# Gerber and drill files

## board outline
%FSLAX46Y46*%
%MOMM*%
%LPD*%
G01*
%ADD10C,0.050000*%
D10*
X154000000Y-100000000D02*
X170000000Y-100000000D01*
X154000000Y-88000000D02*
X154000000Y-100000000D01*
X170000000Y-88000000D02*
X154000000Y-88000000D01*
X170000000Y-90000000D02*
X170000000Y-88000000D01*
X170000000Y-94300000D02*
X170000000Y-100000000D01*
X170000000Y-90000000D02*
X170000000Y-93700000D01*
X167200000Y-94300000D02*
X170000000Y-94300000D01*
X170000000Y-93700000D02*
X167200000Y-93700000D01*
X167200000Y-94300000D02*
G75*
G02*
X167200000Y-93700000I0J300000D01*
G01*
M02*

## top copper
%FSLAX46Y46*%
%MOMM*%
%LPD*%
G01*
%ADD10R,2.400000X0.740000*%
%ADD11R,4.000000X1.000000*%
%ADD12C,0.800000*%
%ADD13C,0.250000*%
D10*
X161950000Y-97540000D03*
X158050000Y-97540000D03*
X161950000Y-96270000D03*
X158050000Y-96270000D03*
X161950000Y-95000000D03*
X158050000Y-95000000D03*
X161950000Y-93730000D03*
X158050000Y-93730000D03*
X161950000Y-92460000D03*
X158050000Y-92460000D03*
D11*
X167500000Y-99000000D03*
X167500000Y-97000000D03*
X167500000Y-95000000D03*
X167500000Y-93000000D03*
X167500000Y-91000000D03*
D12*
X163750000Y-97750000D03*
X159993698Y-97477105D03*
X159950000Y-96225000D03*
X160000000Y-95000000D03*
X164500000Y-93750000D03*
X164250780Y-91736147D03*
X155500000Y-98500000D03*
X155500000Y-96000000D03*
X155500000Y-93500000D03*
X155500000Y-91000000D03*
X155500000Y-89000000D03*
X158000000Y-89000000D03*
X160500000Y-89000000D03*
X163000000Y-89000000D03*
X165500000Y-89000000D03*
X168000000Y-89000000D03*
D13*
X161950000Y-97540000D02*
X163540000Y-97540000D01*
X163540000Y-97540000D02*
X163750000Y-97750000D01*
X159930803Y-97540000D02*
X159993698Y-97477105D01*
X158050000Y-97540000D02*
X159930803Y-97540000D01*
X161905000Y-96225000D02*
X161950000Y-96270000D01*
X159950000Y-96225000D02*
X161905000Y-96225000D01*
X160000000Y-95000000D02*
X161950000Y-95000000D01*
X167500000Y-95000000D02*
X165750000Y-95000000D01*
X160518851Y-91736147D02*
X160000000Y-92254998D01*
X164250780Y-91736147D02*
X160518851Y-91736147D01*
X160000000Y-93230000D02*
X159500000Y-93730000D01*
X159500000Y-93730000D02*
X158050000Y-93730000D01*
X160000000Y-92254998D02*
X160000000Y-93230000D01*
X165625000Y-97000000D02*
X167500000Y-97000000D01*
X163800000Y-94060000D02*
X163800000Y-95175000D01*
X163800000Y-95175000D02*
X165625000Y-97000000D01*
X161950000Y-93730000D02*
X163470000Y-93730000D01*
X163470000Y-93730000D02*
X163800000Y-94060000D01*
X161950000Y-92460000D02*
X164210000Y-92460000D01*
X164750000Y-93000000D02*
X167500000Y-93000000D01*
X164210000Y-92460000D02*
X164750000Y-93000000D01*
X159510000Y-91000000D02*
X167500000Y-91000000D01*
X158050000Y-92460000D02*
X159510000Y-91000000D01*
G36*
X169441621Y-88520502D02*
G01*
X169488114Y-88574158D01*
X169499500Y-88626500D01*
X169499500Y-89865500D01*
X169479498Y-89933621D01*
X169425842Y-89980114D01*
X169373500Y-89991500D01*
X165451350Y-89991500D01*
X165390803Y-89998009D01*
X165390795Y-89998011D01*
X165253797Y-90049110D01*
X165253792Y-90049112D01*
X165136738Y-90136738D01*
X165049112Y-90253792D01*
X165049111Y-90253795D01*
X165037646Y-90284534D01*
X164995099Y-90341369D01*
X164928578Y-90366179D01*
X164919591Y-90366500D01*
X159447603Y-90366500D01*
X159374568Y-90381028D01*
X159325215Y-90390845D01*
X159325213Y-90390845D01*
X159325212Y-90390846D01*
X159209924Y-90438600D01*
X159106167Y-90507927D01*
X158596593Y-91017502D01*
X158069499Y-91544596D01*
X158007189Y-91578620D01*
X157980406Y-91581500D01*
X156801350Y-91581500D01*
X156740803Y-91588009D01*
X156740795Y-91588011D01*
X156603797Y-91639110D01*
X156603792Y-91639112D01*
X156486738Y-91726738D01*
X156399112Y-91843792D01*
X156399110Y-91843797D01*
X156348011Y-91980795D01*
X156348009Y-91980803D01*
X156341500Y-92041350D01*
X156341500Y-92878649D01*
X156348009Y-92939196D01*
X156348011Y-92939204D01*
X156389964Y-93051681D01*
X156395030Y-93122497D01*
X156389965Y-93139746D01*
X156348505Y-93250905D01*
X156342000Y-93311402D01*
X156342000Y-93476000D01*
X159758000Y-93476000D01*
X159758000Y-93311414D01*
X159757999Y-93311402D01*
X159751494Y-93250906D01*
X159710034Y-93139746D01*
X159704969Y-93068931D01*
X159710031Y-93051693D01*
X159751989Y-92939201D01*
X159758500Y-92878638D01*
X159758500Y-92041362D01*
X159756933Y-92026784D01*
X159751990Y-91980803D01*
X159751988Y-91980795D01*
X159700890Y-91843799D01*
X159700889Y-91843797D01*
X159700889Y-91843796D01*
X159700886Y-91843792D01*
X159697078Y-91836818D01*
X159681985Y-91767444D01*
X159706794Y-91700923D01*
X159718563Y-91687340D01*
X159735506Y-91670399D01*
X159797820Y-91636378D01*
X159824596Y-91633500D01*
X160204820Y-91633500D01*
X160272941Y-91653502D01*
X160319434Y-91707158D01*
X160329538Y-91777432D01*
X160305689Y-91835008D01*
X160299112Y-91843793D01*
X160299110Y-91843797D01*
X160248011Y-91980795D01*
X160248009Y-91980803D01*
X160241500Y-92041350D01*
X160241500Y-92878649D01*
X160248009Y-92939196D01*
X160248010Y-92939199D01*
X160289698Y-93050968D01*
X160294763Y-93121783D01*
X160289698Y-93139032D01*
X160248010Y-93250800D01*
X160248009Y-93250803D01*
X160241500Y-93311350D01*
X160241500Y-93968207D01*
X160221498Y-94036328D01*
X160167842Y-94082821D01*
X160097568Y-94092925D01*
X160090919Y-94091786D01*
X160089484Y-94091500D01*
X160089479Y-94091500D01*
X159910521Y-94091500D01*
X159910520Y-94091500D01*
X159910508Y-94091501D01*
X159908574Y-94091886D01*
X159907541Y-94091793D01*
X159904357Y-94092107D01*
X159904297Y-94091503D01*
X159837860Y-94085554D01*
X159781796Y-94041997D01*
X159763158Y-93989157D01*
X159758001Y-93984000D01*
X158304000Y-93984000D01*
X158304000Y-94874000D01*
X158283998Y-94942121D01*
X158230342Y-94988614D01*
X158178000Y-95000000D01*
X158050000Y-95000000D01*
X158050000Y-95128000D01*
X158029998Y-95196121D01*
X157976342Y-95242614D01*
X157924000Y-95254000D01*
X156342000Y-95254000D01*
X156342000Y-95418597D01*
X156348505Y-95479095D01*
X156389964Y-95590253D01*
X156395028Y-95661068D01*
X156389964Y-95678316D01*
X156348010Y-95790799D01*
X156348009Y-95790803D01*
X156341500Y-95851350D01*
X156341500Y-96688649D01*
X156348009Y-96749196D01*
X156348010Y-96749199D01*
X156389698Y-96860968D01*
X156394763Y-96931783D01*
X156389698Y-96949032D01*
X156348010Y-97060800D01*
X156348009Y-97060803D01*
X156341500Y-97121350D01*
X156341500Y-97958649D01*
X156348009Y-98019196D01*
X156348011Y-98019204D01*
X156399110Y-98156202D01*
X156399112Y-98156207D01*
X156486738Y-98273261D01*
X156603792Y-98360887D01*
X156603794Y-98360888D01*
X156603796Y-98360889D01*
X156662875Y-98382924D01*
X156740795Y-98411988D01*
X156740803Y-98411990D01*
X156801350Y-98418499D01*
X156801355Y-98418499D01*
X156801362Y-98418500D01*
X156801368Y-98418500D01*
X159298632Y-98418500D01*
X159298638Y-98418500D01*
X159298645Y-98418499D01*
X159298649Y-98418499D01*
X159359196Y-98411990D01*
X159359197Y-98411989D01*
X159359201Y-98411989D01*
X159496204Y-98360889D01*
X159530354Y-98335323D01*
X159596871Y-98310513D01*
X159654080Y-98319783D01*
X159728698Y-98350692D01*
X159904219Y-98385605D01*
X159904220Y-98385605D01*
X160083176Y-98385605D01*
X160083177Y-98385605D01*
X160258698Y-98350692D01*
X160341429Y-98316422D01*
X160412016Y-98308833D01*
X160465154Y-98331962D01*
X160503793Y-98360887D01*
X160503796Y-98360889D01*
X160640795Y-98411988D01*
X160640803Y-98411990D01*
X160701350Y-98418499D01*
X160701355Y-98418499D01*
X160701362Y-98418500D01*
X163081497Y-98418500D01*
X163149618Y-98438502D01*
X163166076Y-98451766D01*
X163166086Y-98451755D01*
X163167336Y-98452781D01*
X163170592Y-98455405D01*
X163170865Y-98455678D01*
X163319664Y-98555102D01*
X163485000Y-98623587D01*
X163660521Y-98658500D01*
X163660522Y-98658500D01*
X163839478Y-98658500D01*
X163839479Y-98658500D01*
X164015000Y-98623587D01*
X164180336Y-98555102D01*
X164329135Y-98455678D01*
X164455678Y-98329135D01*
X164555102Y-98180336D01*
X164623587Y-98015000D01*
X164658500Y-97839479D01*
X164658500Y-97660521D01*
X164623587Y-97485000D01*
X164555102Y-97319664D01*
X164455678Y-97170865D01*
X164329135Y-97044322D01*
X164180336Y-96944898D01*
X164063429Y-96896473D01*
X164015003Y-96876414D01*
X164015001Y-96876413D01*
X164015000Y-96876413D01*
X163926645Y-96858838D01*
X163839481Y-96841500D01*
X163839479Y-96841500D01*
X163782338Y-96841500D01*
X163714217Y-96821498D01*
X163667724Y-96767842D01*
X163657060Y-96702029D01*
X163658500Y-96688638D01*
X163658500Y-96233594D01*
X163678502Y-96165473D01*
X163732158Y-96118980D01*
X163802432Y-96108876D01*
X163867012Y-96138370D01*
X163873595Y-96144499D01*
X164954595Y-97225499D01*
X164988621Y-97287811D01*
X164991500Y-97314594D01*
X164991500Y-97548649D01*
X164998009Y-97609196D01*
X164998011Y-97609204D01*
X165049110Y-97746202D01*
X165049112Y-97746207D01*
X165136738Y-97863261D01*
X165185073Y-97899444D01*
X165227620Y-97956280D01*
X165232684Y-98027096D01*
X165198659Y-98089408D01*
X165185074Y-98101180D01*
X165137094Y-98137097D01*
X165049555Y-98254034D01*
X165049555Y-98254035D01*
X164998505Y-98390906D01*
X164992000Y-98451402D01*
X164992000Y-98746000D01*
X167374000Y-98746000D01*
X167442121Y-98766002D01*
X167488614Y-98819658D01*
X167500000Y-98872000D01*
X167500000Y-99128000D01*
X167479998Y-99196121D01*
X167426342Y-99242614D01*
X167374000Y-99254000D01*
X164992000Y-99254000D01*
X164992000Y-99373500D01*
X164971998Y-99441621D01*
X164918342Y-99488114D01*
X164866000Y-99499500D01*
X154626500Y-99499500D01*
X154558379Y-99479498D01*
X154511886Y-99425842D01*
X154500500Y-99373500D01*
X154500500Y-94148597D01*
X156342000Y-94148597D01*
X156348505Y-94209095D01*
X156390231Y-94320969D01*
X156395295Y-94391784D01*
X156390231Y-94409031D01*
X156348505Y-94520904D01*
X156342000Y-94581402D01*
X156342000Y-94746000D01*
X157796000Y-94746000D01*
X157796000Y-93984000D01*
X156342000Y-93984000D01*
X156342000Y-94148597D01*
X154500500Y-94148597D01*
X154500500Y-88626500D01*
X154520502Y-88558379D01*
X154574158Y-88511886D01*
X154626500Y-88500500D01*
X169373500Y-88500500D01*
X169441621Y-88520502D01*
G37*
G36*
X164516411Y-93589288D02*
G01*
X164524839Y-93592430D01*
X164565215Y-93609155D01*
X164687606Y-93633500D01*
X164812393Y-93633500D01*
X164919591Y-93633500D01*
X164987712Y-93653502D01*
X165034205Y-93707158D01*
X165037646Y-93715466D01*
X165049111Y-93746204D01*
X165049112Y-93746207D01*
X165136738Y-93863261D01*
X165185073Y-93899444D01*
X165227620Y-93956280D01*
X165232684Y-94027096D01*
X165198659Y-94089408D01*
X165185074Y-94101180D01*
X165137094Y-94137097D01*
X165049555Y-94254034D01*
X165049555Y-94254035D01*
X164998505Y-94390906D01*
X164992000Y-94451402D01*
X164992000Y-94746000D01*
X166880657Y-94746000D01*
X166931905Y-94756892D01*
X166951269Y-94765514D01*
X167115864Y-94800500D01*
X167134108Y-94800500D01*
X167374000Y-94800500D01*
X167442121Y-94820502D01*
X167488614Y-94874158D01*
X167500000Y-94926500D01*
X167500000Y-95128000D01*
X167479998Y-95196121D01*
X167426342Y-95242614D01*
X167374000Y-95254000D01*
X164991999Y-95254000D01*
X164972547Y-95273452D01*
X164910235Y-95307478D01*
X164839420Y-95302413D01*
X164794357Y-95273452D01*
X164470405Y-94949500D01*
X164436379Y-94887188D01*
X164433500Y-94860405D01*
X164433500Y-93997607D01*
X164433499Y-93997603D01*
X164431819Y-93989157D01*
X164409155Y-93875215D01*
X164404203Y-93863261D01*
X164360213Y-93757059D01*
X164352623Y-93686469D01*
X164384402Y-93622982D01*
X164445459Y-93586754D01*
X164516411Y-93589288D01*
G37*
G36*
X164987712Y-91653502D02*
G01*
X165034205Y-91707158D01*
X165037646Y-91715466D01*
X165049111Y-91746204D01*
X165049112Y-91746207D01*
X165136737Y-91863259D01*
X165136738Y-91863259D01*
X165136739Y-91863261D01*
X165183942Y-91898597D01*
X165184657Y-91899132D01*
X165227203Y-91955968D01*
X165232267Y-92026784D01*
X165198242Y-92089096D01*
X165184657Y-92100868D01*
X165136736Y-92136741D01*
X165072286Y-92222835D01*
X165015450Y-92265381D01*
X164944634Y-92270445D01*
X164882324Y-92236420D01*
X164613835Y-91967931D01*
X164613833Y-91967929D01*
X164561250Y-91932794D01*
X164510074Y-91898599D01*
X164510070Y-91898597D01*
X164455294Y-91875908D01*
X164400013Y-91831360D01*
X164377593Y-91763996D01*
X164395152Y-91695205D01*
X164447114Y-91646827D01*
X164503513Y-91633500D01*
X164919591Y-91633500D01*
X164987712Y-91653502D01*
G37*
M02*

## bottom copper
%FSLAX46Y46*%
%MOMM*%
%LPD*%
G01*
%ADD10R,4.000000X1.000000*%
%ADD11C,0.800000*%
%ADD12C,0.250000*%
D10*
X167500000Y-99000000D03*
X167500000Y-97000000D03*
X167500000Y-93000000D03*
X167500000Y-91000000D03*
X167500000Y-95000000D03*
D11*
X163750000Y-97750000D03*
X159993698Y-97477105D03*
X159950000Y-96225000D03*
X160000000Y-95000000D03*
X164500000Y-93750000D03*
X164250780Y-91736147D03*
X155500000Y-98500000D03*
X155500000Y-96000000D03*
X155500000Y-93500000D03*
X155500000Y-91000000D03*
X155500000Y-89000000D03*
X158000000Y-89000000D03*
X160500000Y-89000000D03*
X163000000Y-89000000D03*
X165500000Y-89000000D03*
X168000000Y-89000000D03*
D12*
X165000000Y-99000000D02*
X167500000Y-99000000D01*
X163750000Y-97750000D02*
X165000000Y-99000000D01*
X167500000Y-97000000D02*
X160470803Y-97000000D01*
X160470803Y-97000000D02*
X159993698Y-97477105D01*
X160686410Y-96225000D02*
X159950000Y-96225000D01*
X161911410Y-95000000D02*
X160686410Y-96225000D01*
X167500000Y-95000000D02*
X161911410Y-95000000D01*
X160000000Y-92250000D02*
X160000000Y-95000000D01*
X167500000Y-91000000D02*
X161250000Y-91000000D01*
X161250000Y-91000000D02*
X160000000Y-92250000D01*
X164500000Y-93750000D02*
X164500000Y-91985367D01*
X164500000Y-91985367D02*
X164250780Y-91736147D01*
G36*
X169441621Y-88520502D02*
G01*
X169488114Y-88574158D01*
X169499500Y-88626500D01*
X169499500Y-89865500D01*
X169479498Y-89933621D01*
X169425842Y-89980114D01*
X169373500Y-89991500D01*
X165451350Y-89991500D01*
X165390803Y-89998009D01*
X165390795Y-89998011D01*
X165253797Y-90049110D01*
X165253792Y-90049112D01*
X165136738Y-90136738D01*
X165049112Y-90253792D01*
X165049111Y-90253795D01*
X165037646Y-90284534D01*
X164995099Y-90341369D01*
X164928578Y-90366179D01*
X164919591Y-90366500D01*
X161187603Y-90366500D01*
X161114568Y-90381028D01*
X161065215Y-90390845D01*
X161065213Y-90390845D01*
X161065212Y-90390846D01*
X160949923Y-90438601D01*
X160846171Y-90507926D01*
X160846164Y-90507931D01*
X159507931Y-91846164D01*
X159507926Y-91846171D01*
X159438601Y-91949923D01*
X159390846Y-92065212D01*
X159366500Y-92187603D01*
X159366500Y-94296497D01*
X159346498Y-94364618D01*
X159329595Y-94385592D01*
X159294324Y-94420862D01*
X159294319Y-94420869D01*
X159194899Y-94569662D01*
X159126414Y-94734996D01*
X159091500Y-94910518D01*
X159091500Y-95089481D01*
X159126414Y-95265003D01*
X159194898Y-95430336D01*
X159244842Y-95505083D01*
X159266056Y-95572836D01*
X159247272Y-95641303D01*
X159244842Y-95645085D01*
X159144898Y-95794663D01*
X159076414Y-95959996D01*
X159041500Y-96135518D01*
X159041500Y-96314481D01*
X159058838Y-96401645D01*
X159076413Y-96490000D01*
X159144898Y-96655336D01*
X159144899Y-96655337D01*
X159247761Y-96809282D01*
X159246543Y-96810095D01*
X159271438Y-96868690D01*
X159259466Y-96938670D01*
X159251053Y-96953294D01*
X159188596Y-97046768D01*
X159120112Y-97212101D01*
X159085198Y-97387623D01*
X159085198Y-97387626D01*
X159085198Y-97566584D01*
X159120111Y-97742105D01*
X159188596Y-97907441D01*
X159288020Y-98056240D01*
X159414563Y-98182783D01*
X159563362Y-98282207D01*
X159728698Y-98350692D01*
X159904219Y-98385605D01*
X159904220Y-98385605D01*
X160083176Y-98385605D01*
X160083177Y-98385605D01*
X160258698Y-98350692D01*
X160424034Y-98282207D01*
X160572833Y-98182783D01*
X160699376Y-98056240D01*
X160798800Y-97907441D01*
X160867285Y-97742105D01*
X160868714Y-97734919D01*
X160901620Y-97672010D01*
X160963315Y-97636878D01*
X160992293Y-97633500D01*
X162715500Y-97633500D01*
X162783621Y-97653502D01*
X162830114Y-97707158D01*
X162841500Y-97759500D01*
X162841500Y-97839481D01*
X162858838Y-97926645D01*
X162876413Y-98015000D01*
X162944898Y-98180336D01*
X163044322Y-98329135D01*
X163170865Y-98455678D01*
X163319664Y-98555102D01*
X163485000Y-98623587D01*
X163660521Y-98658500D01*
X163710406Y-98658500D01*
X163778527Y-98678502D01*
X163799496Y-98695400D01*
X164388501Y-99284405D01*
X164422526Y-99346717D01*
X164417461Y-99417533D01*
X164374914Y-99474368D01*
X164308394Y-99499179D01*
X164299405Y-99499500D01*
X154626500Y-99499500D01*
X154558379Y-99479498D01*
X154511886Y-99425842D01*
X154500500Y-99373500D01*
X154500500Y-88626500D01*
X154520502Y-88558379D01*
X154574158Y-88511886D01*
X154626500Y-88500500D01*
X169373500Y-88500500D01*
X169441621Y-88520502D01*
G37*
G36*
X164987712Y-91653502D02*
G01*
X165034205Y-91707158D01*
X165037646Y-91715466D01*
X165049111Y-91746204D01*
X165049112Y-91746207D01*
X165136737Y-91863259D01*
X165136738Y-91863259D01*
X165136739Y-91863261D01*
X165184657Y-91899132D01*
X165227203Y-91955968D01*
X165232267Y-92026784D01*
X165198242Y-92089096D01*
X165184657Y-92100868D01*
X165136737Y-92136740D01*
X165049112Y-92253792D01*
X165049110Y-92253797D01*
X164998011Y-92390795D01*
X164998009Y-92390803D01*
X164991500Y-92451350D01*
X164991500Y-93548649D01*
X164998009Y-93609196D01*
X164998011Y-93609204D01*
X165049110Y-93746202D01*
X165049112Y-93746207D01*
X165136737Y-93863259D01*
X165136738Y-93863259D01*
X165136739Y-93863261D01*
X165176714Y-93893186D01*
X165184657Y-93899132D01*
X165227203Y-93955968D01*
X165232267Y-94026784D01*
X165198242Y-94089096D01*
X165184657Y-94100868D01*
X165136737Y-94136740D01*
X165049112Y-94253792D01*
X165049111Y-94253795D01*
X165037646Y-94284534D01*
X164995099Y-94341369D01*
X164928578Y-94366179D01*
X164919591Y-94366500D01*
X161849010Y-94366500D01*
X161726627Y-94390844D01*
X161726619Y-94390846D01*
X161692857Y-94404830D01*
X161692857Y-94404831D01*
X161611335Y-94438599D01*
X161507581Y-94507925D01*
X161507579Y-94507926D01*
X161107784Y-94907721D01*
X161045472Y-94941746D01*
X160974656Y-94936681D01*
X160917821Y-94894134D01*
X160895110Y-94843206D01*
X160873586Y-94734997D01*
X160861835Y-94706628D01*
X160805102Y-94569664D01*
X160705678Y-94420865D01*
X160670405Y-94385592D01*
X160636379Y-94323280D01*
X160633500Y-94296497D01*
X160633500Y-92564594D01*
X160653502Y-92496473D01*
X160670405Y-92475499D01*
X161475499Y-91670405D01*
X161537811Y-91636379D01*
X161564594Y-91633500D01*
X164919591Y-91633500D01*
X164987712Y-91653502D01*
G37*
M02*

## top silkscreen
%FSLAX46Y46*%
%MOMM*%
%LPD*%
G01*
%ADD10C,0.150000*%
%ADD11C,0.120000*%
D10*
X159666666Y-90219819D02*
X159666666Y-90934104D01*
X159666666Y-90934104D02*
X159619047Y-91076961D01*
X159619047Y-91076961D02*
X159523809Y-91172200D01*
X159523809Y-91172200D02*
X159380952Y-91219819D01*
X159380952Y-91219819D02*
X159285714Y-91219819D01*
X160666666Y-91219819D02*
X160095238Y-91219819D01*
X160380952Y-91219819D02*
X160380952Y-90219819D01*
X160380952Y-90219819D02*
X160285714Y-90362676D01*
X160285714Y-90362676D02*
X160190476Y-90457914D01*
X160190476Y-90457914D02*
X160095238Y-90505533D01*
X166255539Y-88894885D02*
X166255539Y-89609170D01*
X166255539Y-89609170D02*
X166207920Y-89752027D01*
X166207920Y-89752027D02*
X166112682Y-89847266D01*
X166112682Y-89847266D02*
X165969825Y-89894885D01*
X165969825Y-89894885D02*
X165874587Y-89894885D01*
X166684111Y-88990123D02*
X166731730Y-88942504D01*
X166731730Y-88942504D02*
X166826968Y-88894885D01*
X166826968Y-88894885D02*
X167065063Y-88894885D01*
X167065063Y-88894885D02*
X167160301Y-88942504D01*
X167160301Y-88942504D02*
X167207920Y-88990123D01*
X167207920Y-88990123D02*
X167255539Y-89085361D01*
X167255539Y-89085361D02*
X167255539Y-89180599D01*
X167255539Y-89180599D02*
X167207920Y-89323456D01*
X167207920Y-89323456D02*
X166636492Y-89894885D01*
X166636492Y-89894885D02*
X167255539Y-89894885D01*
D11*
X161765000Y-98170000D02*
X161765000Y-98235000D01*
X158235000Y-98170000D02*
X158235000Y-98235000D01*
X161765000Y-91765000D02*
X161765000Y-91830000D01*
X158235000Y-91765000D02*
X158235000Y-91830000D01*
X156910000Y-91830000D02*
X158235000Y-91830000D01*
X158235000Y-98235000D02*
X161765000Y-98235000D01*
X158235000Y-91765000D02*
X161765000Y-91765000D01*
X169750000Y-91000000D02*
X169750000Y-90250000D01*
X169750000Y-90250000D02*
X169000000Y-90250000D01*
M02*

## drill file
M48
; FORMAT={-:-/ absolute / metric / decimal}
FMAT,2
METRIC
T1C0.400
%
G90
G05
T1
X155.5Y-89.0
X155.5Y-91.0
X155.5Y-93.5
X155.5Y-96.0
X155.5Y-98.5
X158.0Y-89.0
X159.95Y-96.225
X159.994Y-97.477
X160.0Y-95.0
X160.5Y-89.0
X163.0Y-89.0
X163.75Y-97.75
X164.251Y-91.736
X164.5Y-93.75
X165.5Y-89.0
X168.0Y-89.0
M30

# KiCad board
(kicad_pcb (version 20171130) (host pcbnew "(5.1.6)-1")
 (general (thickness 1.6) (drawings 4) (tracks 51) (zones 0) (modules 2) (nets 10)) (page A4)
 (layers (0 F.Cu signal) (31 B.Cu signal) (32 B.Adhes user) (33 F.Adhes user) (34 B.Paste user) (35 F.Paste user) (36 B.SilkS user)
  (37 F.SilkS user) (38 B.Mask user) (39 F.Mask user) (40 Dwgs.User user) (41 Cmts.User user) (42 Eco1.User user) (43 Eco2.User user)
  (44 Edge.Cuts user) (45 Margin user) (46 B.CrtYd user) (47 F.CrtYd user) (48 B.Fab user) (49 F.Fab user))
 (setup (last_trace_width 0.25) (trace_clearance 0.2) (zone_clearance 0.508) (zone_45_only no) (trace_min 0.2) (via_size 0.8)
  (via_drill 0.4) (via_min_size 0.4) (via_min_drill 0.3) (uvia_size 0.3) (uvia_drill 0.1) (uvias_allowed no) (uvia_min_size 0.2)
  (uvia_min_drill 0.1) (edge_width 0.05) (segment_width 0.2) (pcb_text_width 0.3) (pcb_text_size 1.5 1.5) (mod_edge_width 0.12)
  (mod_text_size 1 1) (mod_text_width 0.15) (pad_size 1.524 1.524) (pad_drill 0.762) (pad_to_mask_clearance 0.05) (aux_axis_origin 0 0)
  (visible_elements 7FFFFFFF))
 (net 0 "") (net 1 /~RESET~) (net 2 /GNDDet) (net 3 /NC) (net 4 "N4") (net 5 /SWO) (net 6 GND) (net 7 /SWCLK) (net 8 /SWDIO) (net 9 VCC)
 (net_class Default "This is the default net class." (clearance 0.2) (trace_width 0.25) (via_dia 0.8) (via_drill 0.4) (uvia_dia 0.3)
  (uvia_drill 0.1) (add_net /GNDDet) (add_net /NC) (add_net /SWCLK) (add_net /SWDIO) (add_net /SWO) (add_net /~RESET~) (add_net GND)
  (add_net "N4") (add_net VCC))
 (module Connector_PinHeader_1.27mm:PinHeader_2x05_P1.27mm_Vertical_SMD (layer F.Cu) (at 160 95)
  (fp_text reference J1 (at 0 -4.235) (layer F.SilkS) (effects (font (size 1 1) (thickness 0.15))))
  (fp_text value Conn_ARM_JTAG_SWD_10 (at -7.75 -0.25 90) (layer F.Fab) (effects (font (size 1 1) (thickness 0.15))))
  (fp_line (start 1.765 3.17) (end 1.765 3.235) (layer F.SilkS) (width 0.12))
  (fp_line (start -1.765 3.17) (end -1.765 3.235) (layer F.SilkS) (width 0.12))
  (fp_line (start 1.765 -3.235) (end 1.765 -3.17) (layer F.SilkS) (width 0.12))
  (fp_line (start -1.765 -3.235) (end -1.765 -3.17) (layer F.SilkS) (width 0.12))
  (fp_line (start -3.09 -3.17) (end -1.765 -3.17) (layer F.SilkS) (width 0.12))
  (fp_line (start -1.765 3.235) (end 1.765 3.235) (layer F.SilkS) (width 0.12))
  (fp_line (start -1.765 -3.235) (end 1.765 -3.235) (layer F.SilkS) (width 0.12))
  (pad 10 smd rect (at 1.95 2.54) (size 2.4 0.74) (layers F.Cu F.Paste F.Mask) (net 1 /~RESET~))
  (pad 9 smd rect (at -1.95 2.54) (size 2.4 0.74) (layers F.Cu F.Paste F.Mask) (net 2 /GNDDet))
  (pad 8 smd rect (at 1.95 1.27) (size 2.4 0.74) (layers F.Cu F.Paste F.Mask) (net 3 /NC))
  (pad 7 smd rect (at -1.95 1.27) (size 2.4 0.74) (layers F.Cu F.Paste F.Mask) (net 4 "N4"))
  (pad 6 smd rect (at 1.95 0) (size 2.4 0.74) (layers F.Cu F.Paste F.Mask) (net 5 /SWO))
  (pad 5 smd rect (at -1.95 0) (size 2.4 0.74) (layers F.Cu F.Paste F.Mask) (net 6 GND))
  (pad 4 smd rect (at 1.95 -1.27) (size 2.4 0.74) (layers F.Cu F.Paste F.Mask) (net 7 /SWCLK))
  (pad 3 smd rect (at -1.95 -1.27) (size 2.4 0.74) (layers F.Cu F.Paste F.Mask) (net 6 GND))
  (pad 2 smd rect (at 1.95 -2.54) (size 2.4 0.74) (layers F.Cu F.Paste F.Mask) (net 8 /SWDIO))
  (pad 1 smd rect (at -1.95 -2.54) (size 2.4 0.74) (layers F.Cu F.Paste F.Mask) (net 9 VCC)))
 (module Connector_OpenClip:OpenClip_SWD (layer F.Cu) (at 170 95 270)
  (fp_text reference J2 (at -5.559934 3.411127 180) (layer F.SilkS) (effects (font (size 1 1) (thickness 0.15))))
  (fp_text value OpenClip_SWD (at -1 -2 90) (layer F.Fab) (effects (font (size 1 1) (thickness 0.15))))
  (fp_line (start -0.7 0) (end 5 0) (layer Edge.Cuts) (width 0.05))
  (fp_line (start -5 0) (end -1.3 0) (layer Edge.Cuts) (width 0.05))
  (fp_line (start -0.7 2.8) (end -0.7 0) (layer Edge.Cuts) (width 0.05))
  (fp_line (start -1.3 0) (end -1.3 2.8) (layer Edge.Cuts) (width 0.05))
  (fp_line (start -4 0.25) (end -4.75 0.25) (layer F.SilkS) (width 0.12))
  (fp_line (start -4.75 0.25) (end -4.75 1) (layer F.SilkS) (width 0.12))
  (fp_arc (start -1 2.8) (end -1.3 2.8) (angle -180) (layer Edge.Cuts) (width 0.05))
  (pad 5 smd rect (at 4 2.5 270) (size 1 4) (layers F.Cu F.Paste F.Mask) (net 6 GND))
  (pad 4 smd rect (at 2 2.5 270) (size 1 4) (layers F.Cu F.Paste F.Mask) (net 7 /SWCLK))
  (pad 3 smd rect (at 0 2.5 270) (size 1 4) (layers F.Cu F.Paste F.Mask) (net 6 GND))
  (pad 2 smd rect (at -2 2.5 270) (size 1 4) (layers F.Cu F.Paste F.Mask) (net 8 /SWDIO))
  (pad 1 smd rect (at -4 2.5 270) (size 1 4) (layers F.Cu F.Paste F.Mask) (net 9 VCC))
  (pad 10 smd rect (at 4 2.5 270) (size 1 4) (layers B.Cu F.Paste F.Mask) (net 1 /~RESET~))
  (pad 9 smd rect (at 2 2.5 270) (size 1 4) (layers B.Cu F.Paste F.Mask) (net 2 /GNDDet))
  (pad 7 smd rect (at -2 2.5 270) (size 1 4) (layers B.Cu F.Paste F.Mask))
  (pad 6 smd rect (at -4 2.5 270) (size 1 4) (layers B.Cu F.Paste F.Mask) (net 5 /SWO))
  (pad 8 smd rect (at 0 2.5 270) (size 1 4) (layers B.Cu F.Paste F.Mask) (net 3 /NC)))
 (gr_line (start 154 100) (end 170 100) (layer Edge.Cuts) (width 0.05))
 (gr_line (start 154 88) (end 154 100) (layer Edge.Cuts) (width 0.05))
 (gr_line (start 170 88) (end 154 88) (layer Edge.Cuts) (width 0.05))
 (gr_line (start 170 90) (end 170 88) (layer Edge.Cuts) (width 0.05))
 (via (at 163.75 97.75) (size 0.8) (drill 0.4) (layers F.Cu B.Cu) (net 1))
 (segment (start 161.95 97.54) (end 163.54 97.54) (width 0.25) (layer F.Cu) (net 1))
 (segment (start 163.54 97.54) (end 163.75 97.75) (width 0.25) (layer F.Cu) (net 1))
 (segment (start 165 99) (end 167.5 99) (width 0.25) (layer B.Cu) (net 1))
 (segment (start 163.75 97.75) (end 165 99) (width 0.25) (layer B.Cu) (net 1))
 (segment (start 167.5 97) (end 160.470803 97) (width 0.25) (layer B.Cu) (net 2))
 (via (at 159.993698 97.477105) (size 0.8) (drill 0.4) (layers F.Cu B.Cu) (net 2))
 (segment (start 159.930803 97.54) (end 159.993698 97.477105) (width 0.25) (layer F.Cu) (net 2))
 (segment (start 160.470803 97) (end 159.993698 97.477105) (width 0.25) (layer B.Cu) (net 2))
 (segment (start 158.05 97.54) (end 159.930803 97.54) (width 0.25) (layer F.Cu) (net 2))
 (via (at 159.95 96.225) (size 0.8) (drill 0.4) (layers F.Cu B.Cu) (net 3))
 (segment (start 161.905 96.225) (end 161.95 96.27) (width 0.25) (layer F.Cu) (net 3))
 (segment (start 159.95 96.225) (end 161.905 96.225) (width 0.25) (layer F.Cu) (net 3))
 (segment (start 160.68641 96.225) (end 159.95 96.225) (width 0.25) (layer B.Cu) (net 3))
 (segment (start 161.91141 95) (end 160.68641 96.225) (width 0.25) (layer B.Cu) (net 3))
 (segment (start 167.5 95) (end 161.91141 95) (width 0.25) (layer B.Cu) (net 3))
 (via (at 160 95) (size 0.8) (drill 0.4) (layers F.Cu B.Cu) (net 5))
 (segment (start 160 95) (end 161.95 95) (width 0.25) (layer F.Cu) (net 5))
 (segment (start 160 92.25) (end 160 95) (width 0.25) (layer B.Cu) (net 5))
 (segment (start 167.5 91) (end 161.25 91) (width 0.25) (layer B.Cu) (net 5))
 (segment (start 161.25 91) (end 160 92.25) (width 0.25) (layer B.Cu) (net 5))
 (via (at 164.5 93.75) (size 0.8) (drill 0.4) (layers F.Cu B.Cu) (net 6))
 (segment (start 167.5 95) (end 165.75 95) (width 0.25) (layer F.Cu) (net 6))
 (via (at 164.25078 91.736147) (size 0.8) (drill 0.4) (layers F.Cu B.Cu) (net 6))
 (segment (start 164.5 93.75) (end 164.5 91.985367) (width 0.25) (layer B.Cu) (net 6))
 (segment (start 164.5 91.985367) (end 164.25078 91.736147) (width 0.25) (layer B.Cu) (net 6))
 (segment (start 160.518851 91.736147) (end 160 92.254998) (width 0.25) (layer F.Cu) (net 6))
 (segment (start 164.25078 91.736147) (end 160.518851 91.736147) (width 0.25) (layer F.Cu) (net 6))
 (segment (start 160 93.23) (end 159.5 93.73) (width 0.25) (layer F.Cu) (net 6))
 (segment (start 159.5 93.73) (end 158.05 93.73) (width 0.25) (layer F.Cu) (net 6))
 (segment (start 160 92.254998) (end 160 93.23) (width 0.25) (layer F.Cu) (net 6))
 (via (at 155.5 98.5) (size 0.8) (drill 0.4) (layers F.Cu B.Cu) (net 6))
 (via (at 155.5 96) (size 0.8) (drill 0.4) (layers F.Cu B.Cu) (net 6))
 (via (at 155.5 93.5) (size 0.8) (drill 0.4) (layers F.Cu B.Cu) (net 6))
 (via (at 155.5 91) (size 0.8) (drill 0.4) (layers F.Cu B.Cu) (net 6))
 (via (at 155.5 89) (size 0.8) (drill 0.4) (layers F.Cu B.Cu) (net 6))
 (via (at 158 89) (size 0.8) (drill 0.4) (layers F.Cu B.Cu) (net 6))
 (via (at 160.5 89) (size 0.8) (drill 0.4) (layers F.Cu B.Cu) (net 6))
 (via (at 163 89) (size 0.8) (drill 0.4) (layers F.Cu B.Cu) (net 6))
 (via (at 165.5 89) (size 0.8) (drill 0.4) (layers F.Cu B.Cu) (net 6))
 (via (at 168 89) (size 0.8) (drill 0.4) (layers F.Cu B.Cu) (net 6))
 (segment (start 165.625 97) (end 167.5 97) (width 0.25) (layer F.Cu) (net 7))
 (segment (start 163.8 94.06) (end 163.8 95.175) (width 0.25) (layer F.Cu) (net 7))
 (segment (start 163.8 95.175) (end 165.625 97) (width 0.25) (layer F.Cu) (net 7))
 (segment (start 161.95 93.73) (end 163.47 93.73) (width 0.25) (layer F.Cu) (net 7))
 (segment (start 163.47 93.73) (end 163.8 94.06) (width 0.25) (layer F.Cu) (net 7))
 (segment (start 161.95 92.46) (end 164.21 92.46) (width 0.25) (layer F.Cu) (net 8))
 (segment (start 164.75 93) (end 167.5 93) (width 0.25) (layer F.Cu) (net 8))
 (segment (start 164.21 92.46) (end 164.75 93) (width 0.25) (layer F.Cu) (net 8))
 (segment (start 159.51 91) (end 167.5 91) (width 0.25) (layer F.Cu) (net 9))
 (segment (start 158.05 92.46) (end 159.51 91) (width 0.25) (layer F.Cu) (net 9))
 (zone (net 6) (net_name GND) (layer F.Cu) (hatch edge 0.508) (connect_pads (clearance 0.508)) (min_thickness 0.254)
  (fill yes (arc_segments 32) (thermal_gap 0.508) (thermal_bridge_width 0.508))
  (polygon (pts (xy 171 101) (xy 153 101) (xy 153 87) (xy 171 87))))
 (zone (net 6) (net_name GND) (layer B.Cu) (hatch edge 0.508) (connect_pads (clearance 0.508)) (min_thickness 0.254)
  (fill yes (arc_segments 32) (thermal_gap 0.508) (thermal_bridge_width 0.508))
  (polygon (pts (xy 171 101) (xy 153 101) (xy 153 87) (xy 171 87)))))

